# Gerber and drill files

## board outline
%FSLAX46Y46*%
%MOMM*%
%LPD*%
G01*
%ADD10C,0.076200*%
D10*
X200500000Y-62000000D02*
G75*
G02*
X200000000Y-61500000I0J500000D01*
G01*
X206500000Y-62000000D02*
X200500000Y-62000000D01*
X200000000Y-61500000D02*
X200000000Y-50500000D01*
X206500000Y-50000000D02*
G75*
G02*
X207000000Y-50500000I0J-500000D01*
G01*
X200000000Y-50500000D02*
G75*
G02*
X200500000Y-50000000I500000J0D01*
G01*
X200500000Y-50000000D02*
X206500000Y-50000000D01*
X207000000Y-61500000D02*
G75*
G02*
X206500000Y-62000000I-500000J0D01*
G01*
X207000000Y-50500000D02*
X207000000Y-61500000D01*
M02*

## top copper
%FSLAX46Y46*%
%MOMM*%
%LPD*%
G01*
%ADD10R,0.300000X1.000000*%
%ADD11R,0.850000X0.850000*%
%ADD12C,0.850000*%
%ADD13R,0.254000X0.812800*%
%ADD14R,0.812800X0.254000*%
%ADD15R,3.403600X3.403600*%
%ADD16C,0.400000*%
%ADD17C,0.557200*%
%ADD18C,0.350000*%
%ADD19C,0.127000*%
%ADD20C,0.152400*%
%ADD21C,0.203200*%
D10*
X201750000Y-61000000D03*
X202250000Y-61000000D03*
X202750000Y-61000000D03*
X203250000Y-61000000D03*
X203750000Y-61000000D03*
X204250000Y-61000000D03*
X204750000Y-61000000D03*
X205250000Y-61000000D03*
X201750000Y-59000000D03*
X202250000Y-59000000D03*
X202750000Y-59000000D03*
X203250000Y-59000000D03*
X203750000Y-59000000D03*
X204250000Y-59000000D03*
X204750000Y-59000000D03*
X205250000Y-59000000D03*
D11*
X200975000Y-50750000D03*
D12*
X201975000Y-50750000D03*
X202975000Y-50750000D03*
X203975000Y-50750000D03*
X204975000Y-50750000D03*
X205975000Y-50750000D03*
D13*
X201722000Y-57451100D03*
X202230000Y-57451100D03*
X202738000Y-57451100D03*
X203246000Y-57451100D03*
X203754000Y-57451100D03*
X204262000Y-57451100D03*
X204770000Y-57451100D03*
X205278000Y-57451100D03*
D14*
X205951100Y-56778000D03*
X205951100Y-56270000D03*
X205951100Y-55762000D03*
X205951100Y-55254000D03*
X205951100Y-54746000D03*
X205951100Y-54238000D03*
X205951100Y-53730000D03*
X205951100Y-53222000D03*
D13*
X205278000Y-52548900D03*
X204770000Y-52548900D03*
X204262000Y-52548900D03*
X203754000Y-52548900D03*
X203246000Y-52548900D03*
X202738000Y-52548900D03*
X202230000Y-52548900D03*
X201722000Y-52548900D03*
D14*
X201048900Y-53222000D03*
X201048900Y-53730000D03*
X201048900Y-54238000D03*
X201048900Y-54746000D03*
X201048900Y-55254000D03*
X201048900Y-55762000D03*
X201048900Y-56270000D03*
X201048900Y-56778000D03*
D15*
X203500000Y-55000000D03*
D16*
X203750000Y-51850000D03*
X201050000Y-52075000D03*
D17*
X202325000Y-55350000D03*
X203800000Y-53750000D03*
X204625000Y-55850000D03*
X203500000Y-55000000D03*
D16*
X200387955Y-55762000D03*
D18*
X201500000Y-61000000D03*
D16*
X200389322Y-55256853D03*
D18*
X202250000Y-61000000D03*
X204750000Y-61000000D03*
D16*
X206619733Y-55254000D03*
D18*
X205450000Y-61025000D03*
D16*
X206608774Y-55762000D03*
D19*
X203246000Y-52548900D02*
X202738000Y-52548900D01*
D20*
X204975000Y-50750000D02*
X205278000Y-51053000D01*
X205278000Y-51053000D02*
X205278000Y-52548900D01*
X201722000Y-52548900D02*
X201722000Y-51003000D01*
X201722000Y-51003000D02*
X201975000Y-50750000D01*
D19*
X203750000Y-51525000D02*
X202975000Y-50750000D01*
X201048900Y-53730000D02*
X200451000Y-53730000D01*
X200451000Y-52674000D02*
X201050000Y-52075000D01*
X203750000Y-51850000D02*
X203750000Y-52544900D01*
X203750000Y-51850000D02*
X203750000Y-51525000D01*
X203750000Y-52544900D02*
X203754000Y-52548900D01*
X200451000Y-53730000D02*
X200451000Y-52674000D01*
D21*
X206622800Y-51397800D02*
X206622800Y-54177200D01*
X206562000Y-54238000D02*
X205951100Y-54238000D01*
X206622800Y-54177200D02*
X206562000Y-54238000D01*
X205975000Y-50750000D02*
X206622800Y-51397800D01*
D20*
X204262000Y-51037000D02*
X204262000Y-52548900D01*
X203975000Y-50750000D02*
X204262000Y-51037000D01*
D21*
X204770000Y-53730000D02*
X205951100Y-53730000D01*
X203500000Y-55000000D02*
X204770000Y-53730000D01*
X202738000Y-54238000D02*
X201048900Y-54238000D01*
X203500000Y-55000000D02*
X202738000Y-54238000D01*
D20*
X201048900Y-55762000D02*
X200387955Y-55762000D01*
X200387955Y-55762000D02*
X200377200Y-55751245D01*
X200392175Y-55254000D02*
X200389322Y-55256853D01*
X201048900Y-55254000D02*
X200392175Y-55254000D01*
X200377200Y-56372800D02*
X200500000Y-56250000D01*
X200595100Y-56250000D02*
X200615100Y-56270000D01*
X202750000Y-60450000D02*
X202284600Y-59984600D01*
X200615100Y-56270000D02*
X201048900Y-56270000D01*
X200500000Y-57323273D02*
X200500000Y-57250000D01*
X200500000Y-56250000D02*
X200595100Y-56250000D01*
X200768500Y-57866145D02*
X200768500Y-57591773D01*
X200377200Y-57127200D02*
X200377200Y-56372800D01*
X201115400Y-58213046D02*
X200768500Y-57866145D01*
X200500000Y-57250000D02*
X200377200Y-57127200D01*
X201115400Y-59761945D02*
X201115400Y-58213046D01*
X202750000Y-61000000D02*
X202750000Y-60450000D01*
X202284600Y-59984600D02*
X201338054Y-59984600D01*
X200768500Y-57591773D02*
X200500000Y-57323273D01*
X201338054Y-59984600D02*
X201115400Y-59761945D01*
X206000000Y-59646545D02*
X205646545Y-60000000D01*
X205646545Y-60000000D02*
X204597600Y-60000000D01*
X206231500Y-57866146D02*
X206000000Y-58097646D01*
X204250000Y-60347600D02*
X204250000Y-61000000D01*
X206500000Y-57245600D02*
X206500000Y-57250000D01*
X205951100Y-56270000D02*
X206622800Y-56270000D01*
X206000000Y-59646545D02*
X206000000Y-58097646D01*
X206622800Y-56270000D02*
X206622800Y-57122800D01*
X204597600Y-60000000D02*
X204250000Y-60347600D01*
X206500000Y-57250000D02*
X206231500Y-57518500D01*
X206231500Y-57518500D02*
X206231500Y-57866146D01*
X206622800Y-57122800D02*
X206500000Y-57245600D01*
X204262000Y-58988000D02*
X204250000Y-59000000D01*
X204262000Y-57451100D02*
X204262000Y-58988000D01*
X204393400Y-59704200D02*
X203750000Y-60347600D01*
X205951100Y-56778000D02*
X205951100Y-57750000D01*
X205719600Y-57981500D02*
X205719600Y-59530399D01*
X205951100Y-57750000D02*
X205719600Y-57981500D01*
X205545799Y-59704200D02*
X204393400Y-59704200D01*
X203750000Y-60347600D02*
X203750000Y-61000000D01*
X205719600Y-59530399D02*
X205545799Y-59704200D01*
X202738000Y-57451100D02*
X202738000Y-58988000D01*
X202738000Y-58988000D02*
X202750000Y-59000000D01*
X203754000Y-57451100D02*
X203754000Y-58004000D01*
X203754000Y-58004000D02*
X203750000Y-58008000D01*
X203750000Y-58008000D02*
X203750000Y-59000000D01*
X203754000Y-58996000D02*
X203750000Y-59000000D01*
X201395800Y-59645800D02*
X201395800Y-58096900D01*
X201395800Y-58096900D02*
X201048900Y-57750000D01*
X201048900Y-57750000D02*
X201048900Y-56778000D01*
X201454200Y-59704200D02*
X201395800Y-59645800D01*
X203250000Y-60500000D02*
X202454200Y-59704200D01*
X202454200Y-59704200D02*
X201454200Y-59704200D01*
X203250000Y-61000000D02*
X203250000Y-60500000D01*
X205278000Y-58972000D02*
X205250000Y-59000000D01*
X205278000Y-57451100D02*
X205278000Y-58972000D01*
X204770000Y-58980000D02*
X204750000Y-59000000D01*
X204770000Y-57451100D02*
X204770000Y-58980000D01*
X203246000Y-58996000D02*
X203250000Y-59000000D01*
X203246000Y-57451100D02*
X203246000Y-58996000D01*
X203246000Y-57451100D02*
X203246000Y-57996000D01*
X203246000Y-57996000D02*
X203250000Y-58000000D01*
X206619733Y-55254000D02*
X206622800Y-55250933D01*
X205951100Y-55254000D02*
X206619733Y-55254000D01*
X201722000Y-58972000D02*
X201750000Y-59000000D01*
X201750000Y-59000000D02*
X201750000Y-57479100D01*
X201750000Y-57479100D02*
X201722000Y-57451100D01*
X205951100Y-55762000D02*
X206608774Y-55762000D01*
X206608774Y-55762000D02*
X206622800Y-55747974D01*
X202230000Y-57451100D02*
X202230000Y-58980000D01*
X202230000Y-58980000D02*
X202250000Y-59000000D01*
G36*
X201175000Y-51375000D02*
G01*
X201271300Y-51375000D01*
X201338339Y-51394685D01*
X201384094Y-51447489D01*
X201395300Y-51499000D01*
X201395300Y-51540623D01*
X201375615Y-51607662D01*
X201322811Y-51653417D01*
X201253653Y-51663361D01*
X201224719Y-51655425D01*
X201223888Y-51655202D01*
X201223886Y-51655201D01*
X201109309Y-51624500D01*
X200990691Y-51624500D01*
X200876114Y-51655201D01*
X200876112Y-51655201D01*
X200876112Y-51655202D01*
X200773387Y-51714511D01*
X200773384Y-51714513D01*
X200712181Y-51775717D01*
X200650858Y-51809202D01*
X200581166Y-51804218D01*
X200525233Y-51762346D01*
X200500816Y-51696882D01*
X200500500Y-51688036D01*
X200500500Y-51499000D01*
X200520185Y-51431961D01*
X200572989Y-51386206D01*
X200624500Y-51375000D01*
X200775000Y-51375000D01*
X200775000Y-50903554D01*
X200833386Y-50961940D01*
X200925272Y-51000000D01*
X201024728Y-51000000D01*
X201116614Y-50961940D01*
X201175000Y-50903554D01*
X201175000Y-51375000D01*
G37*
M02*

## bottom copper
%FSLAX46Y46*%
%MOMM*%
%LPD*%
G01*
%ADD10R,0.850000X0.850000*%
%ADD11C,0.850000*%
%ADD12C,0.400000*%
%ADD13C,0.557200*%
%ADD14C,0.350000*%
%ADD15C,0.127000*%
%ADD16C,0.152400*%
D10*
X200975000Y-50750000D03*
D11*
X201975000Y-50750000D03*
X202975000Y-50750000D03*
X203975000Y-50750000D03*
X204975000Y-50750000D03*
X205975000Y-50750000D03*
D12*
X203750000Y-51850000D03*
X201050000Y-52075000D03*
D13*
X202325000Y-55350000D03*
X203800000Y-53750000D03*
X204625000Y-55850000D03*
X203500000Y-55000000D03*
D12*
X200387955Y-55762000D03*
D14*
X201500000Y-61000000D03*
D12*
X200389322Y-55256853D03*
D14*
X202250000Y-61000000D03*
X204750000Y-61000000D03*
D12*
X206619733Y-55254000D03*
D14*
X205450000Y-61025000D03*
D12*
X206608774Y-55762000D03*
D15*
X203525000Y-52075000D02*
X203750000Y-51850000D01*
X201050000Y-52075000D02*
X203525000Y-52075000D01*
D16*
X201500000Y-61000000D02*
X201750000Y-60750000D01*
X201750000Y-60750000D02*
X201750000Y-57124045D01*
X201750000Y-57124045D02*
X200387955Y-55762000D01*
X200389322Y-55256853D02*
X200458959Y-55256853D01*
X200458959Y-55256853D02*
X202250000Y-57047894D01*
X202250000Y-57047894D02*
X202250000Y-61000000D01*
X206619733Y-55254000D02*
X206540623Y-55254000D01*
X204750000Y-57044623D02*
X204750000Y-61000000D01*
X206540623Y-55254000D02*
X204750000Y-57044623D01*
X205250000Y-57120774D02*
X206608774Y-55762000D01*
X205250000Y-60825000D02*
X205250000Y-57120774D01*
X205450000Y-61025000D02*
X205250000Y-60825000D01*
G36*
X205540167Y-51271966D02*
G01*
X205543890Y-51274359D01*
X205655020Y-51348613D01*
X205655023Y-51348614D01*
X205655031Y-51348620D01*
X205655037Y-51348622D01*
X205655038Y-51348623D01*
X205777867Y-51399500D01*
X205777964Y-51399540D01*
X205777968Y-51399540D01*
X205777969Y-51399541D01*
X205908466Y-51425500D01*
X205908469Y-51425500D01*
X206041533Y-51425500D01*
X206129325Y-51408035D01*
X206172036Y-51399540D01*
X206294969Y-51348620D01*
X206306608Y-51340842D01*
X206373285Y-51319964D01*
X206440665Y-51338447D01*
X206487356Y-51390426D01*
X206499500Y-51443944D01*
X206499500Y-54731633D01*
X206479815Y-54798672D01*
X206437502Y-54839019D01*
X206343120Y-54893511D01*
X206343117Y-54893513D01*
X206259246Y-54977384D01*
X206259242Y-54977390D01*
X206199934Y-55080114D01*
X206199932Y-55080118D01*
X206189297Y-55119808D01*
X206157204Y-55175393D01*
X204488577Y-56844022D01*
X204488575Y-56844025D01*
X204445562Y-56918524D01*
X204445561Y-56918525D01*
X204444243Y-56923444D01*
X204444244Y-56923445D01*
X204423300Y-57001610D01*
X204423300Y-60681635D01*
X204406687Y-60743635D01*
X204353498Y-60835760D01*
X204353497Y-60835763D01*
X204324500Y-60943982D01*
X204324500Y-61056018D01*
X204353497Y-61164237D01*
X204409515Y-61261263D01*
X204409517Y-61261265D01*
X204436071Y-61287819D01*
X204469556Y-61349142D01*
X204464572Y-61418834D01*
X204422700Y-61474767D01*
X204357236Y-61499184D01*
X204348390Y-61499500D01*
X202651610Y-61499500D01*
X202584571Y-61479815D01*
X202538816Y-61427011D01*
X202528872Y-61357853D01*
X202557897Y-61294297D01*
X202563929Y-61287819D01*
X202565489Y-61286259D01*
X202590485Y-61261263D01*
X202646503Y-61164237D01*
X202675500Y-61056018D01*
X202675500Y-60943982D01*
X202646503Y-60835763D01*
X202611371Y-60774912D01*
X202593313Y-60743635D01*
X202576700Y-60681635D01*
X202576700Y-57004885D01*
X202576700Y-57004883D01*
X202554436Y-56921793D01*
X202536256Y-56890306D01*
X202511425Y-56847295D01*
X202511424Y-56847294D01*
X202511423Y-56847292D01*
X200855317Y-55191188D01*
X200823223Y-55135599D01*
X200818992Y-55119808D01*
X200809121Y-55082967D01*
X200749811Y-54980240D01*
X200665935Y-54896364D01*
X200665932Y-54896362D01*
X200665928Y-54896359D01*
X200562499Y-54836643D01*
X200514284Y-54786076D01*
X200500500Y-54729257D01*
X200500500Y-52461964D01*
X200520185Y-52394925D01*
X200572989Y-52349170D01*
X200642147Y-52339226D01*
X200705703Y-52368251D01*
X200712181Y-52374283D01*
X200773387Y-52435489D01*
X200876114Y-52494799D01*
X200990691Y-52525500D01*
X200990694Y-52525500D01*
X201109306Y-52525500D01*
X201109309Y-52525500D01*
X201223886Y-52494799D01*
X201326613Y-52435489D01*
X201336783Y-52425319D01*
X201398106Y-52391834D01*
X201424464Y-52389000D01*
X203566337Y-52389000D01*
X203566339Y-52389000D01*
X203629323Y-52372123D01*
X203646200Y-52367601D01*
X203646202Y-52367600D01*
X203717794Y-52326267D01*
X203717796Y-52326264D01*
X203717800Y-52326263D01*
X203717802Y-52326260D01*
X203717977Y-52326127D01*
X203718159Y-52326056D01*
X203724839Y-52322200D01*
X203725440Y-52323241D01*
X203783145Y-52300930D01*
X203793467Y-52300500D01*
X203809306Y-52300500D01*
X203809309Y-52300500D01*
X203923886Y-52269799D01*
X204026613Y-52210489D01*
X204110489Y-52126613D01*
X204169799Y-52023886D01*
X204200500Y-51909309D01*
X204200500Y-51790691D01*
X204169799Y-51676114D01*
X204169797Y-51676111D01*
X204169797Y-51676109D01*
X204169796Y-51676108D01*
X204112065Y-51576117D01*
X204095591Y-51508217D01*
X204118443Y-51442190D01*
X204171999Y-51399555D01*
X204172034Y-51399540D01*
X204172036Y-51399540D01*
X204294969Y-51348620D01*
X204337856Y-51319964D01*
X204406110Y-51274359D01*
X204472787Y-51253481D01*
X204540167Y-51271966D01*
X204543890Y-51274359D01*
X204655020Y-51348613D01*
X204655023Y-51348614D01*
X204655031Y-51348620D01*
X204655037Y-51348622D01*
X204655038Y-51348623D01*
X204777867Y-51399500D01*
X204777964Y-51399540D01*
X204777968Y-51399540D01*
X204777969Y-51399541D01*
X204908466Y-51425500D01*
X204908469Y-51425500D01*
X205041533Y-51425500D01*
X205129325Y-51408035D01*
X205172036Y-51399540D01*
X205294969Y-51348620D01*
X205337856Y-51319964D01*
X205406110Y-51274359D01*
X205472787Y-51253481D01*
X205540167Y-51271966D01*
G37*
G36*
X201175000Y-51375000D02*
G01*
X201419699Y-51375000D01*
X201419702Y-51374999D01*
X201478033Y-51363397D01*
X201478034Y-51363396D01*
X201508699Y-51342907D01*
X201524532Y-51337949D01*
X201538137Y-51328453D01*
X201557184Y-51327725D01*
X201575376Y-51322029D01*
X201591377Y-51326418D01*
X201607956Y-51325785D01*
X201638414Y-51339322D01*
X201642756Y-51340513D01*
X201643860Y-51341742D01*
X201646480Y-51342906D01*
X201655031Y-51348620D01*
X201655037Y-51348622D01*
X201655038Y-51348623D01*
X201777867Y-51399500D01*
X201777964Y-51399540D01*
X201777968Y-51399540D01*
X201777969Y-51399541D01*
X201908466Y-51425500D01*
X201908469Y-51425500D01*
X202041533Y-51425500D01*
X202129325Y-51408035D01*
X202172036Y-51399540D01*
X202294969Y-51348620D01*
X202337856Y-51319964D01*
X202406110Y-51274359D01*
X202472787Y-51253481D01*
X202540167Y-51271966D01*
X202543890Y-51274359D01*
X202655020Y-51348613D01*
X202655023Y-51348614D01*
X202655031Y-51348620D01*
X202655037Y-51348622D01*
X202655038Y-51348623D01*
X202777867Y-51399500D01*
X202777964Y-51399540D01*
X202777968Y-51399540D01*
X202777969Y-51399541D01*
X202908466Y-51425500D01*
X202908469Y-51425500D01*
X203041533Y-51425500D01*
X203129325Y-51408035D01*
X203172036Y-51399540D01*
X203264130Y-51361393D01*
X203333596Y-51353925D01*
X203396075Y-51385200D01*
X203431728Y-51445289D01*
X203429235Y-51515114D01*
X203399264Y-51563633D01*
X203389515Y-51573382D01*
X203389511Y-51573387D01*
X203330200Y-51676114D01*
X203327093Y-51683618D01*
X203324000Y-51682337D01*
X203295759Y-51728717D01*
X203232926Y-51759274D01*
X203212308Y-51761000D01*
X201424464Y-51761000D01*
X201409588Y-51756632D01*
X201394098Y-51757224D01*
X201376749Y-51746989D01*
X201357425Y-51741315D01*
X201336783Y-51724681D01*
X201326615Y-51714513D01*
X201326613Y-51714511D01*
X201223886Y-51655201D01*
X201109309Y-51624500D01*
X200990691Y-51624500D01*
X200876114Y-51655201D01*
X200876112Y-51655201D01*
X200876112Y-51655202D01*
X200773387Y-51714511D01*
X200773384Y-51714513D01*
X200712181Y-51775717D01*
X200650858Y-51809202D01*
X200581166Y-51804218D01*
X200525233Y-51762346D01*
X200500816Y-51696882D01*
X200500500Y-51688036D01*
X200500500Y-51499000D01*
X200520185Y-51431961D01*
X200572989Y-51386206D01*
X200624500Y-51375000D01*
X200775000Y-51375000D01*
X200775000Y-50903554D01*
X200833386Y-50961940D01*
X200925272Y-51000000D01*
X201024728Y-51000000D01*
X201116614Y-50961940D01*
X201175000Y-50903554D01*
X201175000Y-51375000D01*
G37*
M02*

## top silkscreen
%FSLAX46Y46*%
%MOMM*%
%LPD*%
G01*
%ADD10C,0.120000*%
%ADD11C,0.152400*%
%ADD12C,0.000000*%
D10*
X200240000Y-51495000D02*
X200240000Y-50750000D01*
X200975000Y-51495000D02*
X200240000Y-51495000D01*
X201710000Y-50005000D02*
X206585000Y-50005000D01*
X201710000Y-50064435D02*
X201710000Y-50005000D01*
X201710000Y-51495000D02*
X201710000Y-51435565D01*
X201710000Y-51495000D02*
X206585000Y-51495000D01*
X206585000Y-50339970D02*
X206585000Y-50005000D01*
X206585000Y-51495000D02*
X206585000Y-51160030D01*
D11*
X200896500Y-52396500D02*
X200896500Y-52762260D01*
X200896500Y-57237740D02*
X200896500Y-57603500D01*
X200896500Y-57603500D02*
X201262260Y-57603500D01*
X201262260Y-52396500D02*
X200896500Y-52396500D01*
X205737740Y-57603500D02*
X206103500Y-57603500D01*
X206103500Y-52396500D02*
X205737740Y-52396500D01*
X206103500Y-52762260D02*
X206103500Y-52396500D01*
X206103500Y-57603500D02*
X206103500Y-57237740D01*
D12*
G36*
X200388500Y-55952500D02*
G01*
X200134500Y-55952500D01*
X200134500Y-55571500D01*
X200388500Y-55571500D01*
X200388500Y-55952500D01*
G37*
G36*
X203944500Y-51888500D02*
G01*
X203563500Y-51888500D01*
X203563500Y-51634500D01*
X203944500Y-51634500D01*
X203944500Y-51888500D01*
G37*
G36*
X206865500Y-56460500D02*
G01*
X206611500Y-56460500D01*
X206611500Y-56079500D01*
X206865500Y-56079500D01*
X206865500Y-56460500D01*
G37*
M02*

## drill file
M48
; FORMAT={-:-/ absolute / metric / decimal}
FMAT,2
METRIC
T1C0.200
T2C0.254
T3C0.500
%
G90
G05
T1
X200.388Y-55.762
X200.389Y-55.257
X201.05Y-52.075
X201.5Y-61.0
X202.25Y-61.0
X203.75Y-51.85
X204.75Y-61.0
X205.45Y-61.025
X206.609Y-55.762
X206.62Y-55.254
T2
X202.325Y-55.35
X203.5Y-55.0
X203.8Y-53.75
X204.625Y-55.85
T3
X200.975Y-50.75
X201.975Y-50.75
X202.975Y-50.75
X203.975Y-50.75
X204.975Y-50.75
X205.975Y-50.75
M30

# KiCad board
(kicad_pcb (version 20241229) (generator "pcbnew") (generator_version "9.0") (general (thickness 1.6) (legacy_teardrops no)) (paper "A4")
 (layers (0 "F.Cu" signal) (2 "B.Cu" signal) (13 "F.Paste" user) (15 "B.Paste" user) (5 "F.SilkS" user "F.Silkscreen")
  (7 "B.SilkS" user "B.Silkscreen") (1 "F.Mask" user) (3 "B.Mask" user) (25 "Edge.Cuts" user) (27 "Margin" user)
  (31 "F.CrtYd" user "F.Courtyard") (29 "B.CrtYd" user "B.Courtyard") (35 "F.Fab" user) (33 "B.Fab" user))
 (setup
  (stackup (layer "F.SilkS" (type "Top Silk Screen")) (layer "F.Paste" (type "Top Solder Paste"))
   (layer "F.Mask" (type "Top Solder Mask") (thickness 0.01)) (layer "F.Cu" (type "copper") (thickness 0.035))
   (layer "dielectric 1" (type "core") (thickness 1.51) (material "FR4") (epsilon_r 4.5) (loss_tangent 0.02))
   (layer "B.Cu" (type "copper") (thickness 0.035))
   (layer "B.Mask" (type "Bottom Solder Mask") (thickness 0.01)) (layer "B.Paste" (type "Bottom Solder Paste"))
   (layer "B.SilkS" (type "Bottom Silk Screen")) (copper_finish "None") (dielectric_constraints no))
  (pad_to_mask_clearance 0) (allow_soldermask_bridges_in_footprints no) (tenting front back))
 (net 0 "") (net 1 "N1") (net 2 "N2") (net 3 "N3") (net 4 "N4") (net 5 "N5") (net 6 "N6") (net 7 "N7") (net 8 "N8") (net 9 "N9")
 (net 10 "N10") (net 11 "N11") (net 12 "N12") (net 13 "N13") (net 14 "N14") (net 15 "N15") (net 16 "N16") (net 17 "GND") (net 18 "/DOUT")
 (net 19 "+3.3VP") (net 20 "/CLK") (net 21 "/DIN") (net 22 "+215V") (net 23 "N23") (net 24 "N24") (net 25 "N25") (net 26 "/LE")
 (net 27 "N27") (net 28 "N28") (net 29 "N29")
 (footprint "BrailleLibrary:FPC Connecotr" (layer "F.Cu") (at 203.5 61 90)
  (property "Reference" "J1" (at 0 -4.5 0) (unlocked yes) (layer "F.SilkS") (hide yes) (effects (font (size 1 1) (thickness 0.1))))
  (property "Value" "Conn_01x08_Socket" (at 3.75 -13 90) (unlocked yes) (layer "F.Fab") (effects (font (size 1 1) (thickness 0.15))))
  (pad "1" smd rect (at 0 -1.75 90) (size 1 0.3) (layers "F.Cu" "F.Mask" "F.Paste") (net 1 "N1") (thermal_bridge_angle 45))
  (pad "2" smd rect (at 0 -1.25 90) (size 1 0.3) (layers "F.Cu" "F.Mask" "F.Paste") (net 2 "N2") (thermal_bridge_angle 45))
  (pad "3" smd rect (at 0 -0.75 90) (size 1 0.3) (layers "F.Cu" "F.Mask" "F.Paste") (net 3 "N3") (thermal_bridge_angle 45))
  (pad "4" smd rect (at 0 -0.25 90) (size 1 0.3) (layers "F.Cu" "F.Mask" "F.Paste") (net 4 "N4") (thermal_bridge_angle 45))
  (pad "5" smd rect (at 0 0.25 90) (size 1 0.3) (layers "F.Cu" "F.Mask" "F.Paste") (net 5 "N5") (thermal_bridge_angle 45))
  (pad "6" smd rect (at 0 0.75 90) (size 1 0.3) (layers "F.Cu" "F.Mask" "F.Paste") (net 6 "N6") (thermal_bridge_angle 45))
  (pad "7" smd rect (at 0 1.25 90) (size 1 0.3) (layers "F.Cu" "F.Mask" "F.Paste") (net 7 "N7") (thermal_bridge_angle 45))
  (pad "8" smd rect (at 0 1.75 90) (size 1 0.3) (layers "F.Cu" "F.Mask" "F.Paste") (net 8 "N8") (thermal_bridge_angle 45)))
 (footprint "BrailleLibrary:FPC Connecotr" (layer "F.Cu") (at 203.5 59 90)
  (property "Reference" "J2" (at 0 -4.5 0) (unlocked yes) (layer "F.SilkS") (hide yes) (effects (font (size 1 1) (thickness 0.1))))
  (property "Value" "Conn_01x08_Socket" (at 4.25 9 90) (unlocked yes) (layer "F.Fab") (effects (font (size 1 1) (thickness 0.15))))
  (pad "1" smd rect (at 0 -1.75 90) (size 1 0.3) (layers "F.Cu" "F.Mask" "F.Paste") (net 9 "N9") (thermal_bridge_angle 45))
  (pad "2" smd rect (at 0 -1.25 90) (size 1 0.3) (layers "F.Cu" "F.Mask" "F.Paste") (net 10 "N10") (thermal_bridge_angle 45))
  (pad "3" smd rect (at 0 -0.75 90) (size 1 0.3) (layers "F.Cu" "F.Mask" "F.Paste") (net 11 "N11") (thermal_bridge_angle 45))
  (pad "4" smd rect (at 0 -0.25 90) (size 1 0.3) (layers "F.Cu" "F.Mask" "F.Paste") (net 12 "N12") (thermal_bridge_angle 45))
  (pad "5" smd rect (at 0 0.25 90) (size 1 0.3) (layers "F.Cu" "F.Mask" "F.Paste") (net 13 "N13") (thermal_bridge_angle 45))
  (pad "6" smd rect (at 0 0.75 90) (size 1 0.3) (layers "F.Cu" "F.Mask" "F.Paste") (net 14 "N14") (thermal_bridge_angle 45))
  (pad "7" smd rect (at 0 1.25 90) (size 1 0.3) (layers "F.Cu" "F.Mask" "F.Paste") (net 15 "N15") (thermal_bridge_angle 45))
  (pad "8" smd rect (at 0 1.75 90) (size 1 0.3) (layers "F.Cu" "F.Mask" "F.Paste") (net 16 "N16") (thermal_bridge_angle 45)))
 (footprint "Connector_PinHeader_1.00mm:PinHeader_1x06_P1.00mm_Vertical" (layer "F.Cu") (at 200.975 50.75 90)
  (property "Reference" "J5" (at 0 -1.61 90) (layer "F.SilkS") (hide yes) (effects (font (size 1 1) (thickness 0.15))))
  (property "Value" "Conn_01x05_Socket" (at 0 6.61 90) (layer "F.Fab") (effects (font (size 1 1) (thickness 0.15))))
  (fp_line (start -0.745 -0.735) (end 0 -0.735) (stroke (width 0.12) (type solid)) (layer "F.SilkS"))
  (fp_line (start -0.745 0) (end -0.745 -0.735) (stroke (width 0.12) (type solid)) (layer "F.SilkS"))
  (fp_line (start 0.745 0.735) (end 0.745 5.61) (stroke (width 0.12) (type solid)) (layer "F.SilkS"))
  (fp_line (start 0.685565 0.735) (end 0.745 0.735) (stroke (width 0.12) (type solid)) (layer "F.SilkS"))
  (fp_line (start -0.745 0.735) (end -0.685565 0.735) (stroke (width 0.12) (type solid)) (layer "F.SilkS"))
  (fp_line (start -0.745 0.735) (end -0.745 5.61) (stroke (width 0.12) (type solid)) (layer "F.SilkS"))
  (fp_line (start 0.41003 5.61) (end 0.745 5.61) (stroke (width 0.12) (type solid)) (layer "F.SilkS"))
  (fp_line (start -0.745 5.61) (end -0.41003 5.61) (stroke (width 0.12) (type solid)) (layer "F.SilkS"))
  (pad "1" thru_hole rect (at 0 0 90) (size 0.85 0.85) (drill 0.5) (layers "*.Cu" "*.Mask") (remove_unused_layers no) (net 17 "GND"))
  (pad "2" thru_hole circle (at 0 1 90) (size 0.85 0.85) (drill 0.5) (layers "*.Cu" "*.Mask") (remove_unused_layers no) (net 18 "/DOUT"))
  (pad "3" thru_hole circle (at 0 2 90) (size 0.85 0.85) (drill 0.5) (layers "*.Cu" "*.Mask") (remove_unused_layers no) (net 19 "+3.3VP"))
  (pad "4" thru_hole circle (at 0 3 90) (size 0.85 0.85) (drill 0.5) (layers "*.Cu" "*.Mask") (remove_unused_layers no) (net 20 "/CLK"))
  (pad "5" thru_hole circle (at 0 4 90) (size 0.85 0.85) (drill 0.5) (layers "*.Cu" "*.Mask") (remove_unused_layers no) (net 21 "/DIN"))
  (pad "6" thru_hole circle (at 0 5 90) (size 0.85 0.85) (drill 0.5) (layers "*.Cu" "*.Mask") (remove_unused_layers no) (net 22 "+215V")))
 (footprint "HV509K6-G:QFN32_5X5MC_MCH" (layer "F.Cu") (at 203.5 55 90)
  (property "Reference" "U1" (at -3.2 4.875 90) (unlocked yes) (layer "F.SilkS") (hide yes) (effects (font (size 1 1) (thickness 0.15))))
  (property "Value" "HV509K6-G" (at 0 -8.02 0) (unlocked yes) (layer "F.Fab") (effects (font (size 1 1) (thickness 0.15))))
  (fp_line (start 2.6035 -2.6035) (end 2.23774 -2.6035) (stroke (width 0.1524) (type solid)) (layer "F.SilkS"))
  (fp_line (start -2.23774 -2.6035) (end -2.6035 -2.6035) (stroke (width 0.1524) (type solid)) (layer "F.SilkS"))
  (fp_line (start -2.6035 -2.6035) (end -2.6035 -2.23774) (stroke (width 0.1524) (type solid)) (layer "F.SilkS"))
  (fp_line (start 2.6035 -2.23774) (end 2.6035 -2.6035) (stroke (width 0.1524) (type solid)) (layer "F.SilkS"))
  (fp_line (start -2.6035 2.23774) (end -2.6035 2.6035) (stroke (width 0.1524) (type solid)) (layer "F.SilkS"))
  (fp_line (start 2.6035 2.6035) (end 2.6035 2.23774) (stroke (width 0.1524) (type solid)) (layer "F.SilkS"))
  (fp_line (start 2.23774 2.6035) (end 2.6035 2.6035) (stroke (width 0.1524) (type solid)) (layer "F.SilkS"))
  (fp_line (start -2.6035 2.6035) (end -2.23774 2.6035) (stroke (width 0.1524) (type solid)) (layer "F.SilkS"))
  (fp_poly
   (pts (xy -0.9525 -3.1115) (xy -0.9525 -3.3655) (xy -0.5715 -3.3655) (xy -0.5715 -3.1115)) (stroke (width 0) (type solid)) (fill yes)
   (layer "F.SilkS"))
  (fp_poly
   (pts (xy 3.3655 0.0635) (xy 3.3655 0.4445) (xy 3.1115 0.4445) (xy 3.1115 0.0635)) (stroke (width 0) (type solid)) (fill yes)
   (layer "F.SilkS"))
  (fp_poly
   (pts (xy -1.4605 3.1115) (xy -1.4605 3.3655) (xy -1.0795 3.3655) (xy -1.0795 3.1115)) (stroke (width 0) (type solid)) (fill yes)
   (layer "F.SilkS"))
  (pad "1" smd rect (at -2.4511 -1.778 180) (size 0.254 0.8128) (layers "F.Cu" "F.Mask" "F.Paste") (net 9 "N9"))
  (pad "2" smd rect (at -2.4511 -1.27 180) (size 0.254 0.8128) (layers "F.Cu" "F.Mask" "F.Paste") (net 10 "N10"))
  (pad "3" smd rect (at -2.4511 -0.762 180) (size 0.254 0.8128) (layers "F.Cu" "F.Mask" "F.Paste") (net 11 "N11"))
  (pad "4" smd rect (at -2.4511 -0.254 180) (size 0.254 0.8128) (layers "F.Cu" "F.Mask" "F.Paste") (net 12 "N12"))
  (pad "5" smd rect (at -2.4511 0.254 180) (size 0.254 0.8128) (layers "F.Cu" "F.Mask" "F.Paste") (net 13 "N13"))
  (pad "6" smd rect (at -2.4511 0.762 180) (size 0.254 0.8128) (layers "F.Cu" "F.Mask" "F.Paste") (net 14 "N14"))
  (pad "7" smd rect (at -2.4511 1.27 180) (size 0.254 0.8128) (layers "F.Cu" "F.Mask" "F.Paste") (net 15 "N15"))
  (pad "8" smd rect (at -2.4511 1.778 180) (size 0.254 0.8128) (layers "F.Cu" "F.Mask" "F.Paste") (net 16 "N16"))
  (pad "9" smd rect (at -1.778 2.4511 90) (size 0.254 0.8128) (layers "F.Cu" "F.Mask" "F.Paste") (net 5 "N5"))
  (pad "10" smd rect (at -1.27 2.4511 90) (size 0.254 0.8128) (layers "F.Cu" "F.Mask" "F.Paste") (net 6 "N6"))
  (pad "11" smd rect (at -0.762 2.4511 90) (size 0.254 0.8128) (layers "F.Cu" "F.Mask" "F.Paste") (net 8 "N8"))
  (pad "12" smd rect (at -0.254 2.4511 90) (size 0.254 0.8128) (layers "F.Cu" "F.Mask" "F.Paste") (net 7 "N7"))
  (pad "13" smd rect (at 0.254 2.4511 90) (size 0.254 0.8128) (layers "F.Cu" "F.Mask" "F.Paste") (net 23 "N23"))
  (pad "14" smd rect (at 0.762 2.4511 90) (size 0.254 0.8128) (layers "F.Cu" "F.Mask" "F.Paste") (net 22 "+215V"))
  (pad "15" smd rect (at 1.27 2.4511 90) (size 0.254 0.8128) (layers "F.Cu" "F.Mask" "F.Paste") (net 17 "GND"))
  (pad "16" smd rect (at 1.778 2.4511 90) (size 0.254 0.8128) (layers "F.Cu" "F.Mask" "F.Paste") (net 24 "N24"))
  (pad "17" smd rect (at 2.4511 1.778 180) (size 0.254 0.8128) (layers "F.Cu" "F.Mask" "F.Paste") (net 21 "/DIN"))
  (pad "18" smd rect (at 2.4511 1.27 180) (size 0.254 0.8128) (layers "F.Cu" "F.Mask" "F.Paste") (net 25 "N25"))
  (pad "19" smd rect (at 2.4511 0.762 180) (size 0.254 0.8128) (layers "F.Cu" "F.Mask" "F.Paste") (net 20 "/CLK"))
  (pad "20" smd rect (at 2.4511 0.254 180) (size 0.254 0.8128) (layers "F.Cu" "F.Mask" "F.Paste") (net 19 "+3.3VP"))
  (pad "21" smd rect (at 2.4511 -0.254 180) (size 0.254 0.8128) (layers "F.Cu" "F.Mask" "F.Paste") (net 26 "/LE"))
  (pad "22" smd rect (at 2.4511 -0.762 180) (size 0.254 0.8128) (layers "F.Cu" "F.Mask" "F.Paste") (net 26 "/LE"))
  (pad "23" smd rect (at 2.4511 -1.27 180) (size 0.254 0.8128) (layers "F.Cu" "F.Mask" "F.Paste") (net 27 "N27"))
  (pad "24" smd rect (at 2.4511 -1.778 180) (size 0.254 0.8128) (layers "F.Cu" "F.Mask" "F.Paste") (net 18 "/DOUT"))
  (pad "25" smd rect (at 1.778 -2.4511 90) (size 0.254 0.8128) (layers "F.Cu" "F.Mask" "F.Paste") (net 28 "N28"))
  (pad "26" smd rect (at 1.27 -2.4511 90) (size 0.254 0.8128) (layers "F.Cu" "F.Mask" "F.Paste") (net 19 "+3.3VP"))
  (pad "27" smd rect (at 0.762 -2.4511 90) (size 0.254 0.8128) (layers "F.Cu" "F.Mask" "F.Paste") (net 17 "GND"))
  (pad "28" smd rect (at 0.254 -2.4511 90) (size 0.254 0.8128) (layers "F.Cu" "F.Mask" "F.Paste") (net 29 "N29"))
  (pad "29" smd rect (at -0.254 -2.4511 90) (size 0.254 0.8128) (layers "F.Cu" "F.Mask" "F.Paste") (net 2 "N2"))
  (pad "30" smd rect (at -0.762 -2.4511 90) (size 0.254 0.8128) (layers "F.Cu" "F.Mask" "F.Paste") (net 1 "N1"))
  (pad "31" smd rect (at -1.27 -2.4511 90) (size 0.254 0.8128) (layers "F.Cu" "F.Mask" "F.Paste") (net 3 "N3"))
  (pad "32" smd rect (at -1.778 -2.4511 90) (size 0.254 0.8128) (layers "F.Cu" "F.Mask" "F.Paste") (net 4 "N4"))
  (pad "33" smd rect (at 0 0 90) (size 3.4036 3.4036) (layers "F.Cu" "F.Mask" "F.Paste") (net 17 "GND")))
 (gr_arc (start 200.5 62) (mid 200.146447 61.853553) (end 200 61.5) (stroke (width 0.0762) (type default)) (layer "Edge.Cuts"))
 (gr_line (start 206.5 62) (end 200.5 62) (stroke (width 0.0762) (type default)) (layer "Edge.Cuts"))
 (gr_line (start 200 61.5) (end 200 50.5) (stroke (width 0.0762) (type default)) (layer "Edge.Cuts"))
 (gr_arc (start 206.5 50) (mid 206.853553 50.146447) (end 207 50.5) (stroke (width 0.0762) (type default)) (layer "Edge.Cuts"))
 (gr_arc (start 200 50.5) (mid 200.146447 50.146447) (end 200.5 50) (stroke (width 0.0762) (type default)) (layer "Edge.Cuts"))
 (gr_line (start 200.5 50) (end 206.5 50) (stroke (width 0.0762) (type default)) (layer "Edge.Cuts"))
 (gr_arc (start 207 61.5) (mid 206.853553 61.853553) (end 206.5 62) (stroke (width 0.0762) (type default)) (layer "Edge.Cuts"))
 (gr_line (start 207 50.5) (end 207 61.5) (stroke (width 0.0762) (type default)) (layer "Edge.Cuts"))
 (segment (start 203.246 52.5489) (end 202.738 52.5489) (width 0.127) (layer "F.Cu") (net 26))
 (segment (start 204.975 50.75) (end 205.278 51.053) (width 0.1524) (layer "F.Cu") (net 21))
 (segment (start 205.278 51.053) (end 205.278 52.5489) (width 0.1524) (layer "F.Cu") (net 21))
 (segment (start 201.722 52.5489) (end 201.722 51.003) (width 0.1524) (layer "F.Cu") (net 18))
 (segment (start 201.722 51.003) (end 201.975 50.75) (width 0.1524) (layer "F.Cu") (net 18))
 (segment (start 203.75 51.525) (end 202.975 50.75) (width 0.127) (layer "F.Cu") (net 19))
 (segment (start 201.0489 53.73) (end 200.451 53.73) (width 0.127) (layer "F.Cu") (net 19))
 (segment (start 200.451 52.674) (end 201.05 52.075) (width 0.127) (layer "F.Cu") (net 19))
 (segment (start 203.75 51.85) (end 203.75 52.5449) (width 0.127) (layer "F.Cu") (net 19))
 (segment (start 203.75 51.85) (end 203.75 51.525) (width 0.127) (layer "F.Cu") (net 19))
 (segment (start 203.75 52.5449) (end 203.754 52.5489) (width 0.127) (layer "F.Cu") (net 19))
 (segment (start 200.451 53.73) (end 200.451 52.674) (width 0.127) (layer "F.Cu") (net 19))
 (via (at 203.75 51.85) (size 0.4) (drill 0.2) (layers "F.Cu" "B.Cu") (free yes) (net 19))
 (via (at 201.05 52.075) (size 0.4) (drill 0.2) (layers "F.Cu" "B.Cu") (free yes) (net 19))
 (segment (start 203.525 52.075) (end 203.75 51.85) (width 0.127) (layer "B.Cu") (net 19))
 (segment (start 201.05 52.075) (end 203.525 52.075) (width 0.127) (layer "B.Cu") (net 19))
 (segment (start 206.6228 51.3978) (end 206.6228 54.1772) (width 0.2032) (layer "F.Cu") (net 22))
 (segment (start 206.562 54.238) (end 205.9511 54.238) (width 0.2032) (layer "F.Cu") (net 22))
 (segment (start 206.6228 54.1772) (end 206.562 54.238) (width 0.2032) (layer "F.Cu") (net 22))
 (segment (start 205.975 50.75) (end 206.6228 51.3978) (width 0.2032) (layer "F.Cu") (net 22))
 (segment (start 204.262 51.037) (end 204.262 52.5489) (width 0.1524) (layer "F.Cu") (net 20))
 (segment (start 203.975 50.75) (end 204.262 51.037) (width 0.1524) (layer "F.Cu") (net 20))
 (segment (start 204.77 53.73) (end 205.9511 53.73) (width 0.2032) (layer "F.Cu") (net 17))
 (segment (start 203.5 55) (end 204.77 53.73) (width 0.2032) (layer "F.Cu") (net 17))
 (segment (start 202.738 54.238) (end 201.0489 54.238) (width 0.2032) (layer "F.Cu") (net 17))
 (segment (start 203.5 55) (end 202.738 54.238) (width 0.2032) (layer "F.Cu") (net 17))
 (via (at 202.325 55.35) (size 0.5572) (drill 0.254) (layers "F.Cu" "B.Cu") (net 17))
 (via (at 203.8 53.75) (size 0.5572) (drill 0.254) (layers "F.Cu" "B.Cu") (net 17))
 (via (at 204.625 55.85) (size 0.5572) (drill 0.254) (layers "F.Cu" "B.Cu") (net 17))
 (via (at 203.5 55) (size 0.5572) (drill 0.254) (layers "F.Cu" "B.Cu") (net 17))
 (segment (start 201.0489 55.762) (end 200.387955 55.762) (width 0.1524) (layer "F.Cu") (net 1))
 (segment (start 200.387955 55.762) (end 200.3772 55.751245) (width 0.1524) (layer "F.Cu") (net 1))
 (via (at 200.387955 55.762) (size 0.4) (drill 0.2) (layers "F.Cu" "B.Cu") (free yes) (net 1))
 (via (at 201.5 61) (size 0.35) (drill 0.2) (layers "F.Cu" "B.Cu") (free yes) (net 1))
 (segment (start 201.5 61) (end 201.75 60.75) (width 0.1524) (layer "B.Cu") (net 1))
 (segment (start 201.75 60.75) (end 201.75 57.124045) (width 0.1524) (layer "B.Cu") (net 1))
 (segment (start 201.75 57.124045) (end 200.387955 55.762) (width 0.1524) (layer "B.Cu") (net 1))
 (segment (start 200.392175 55.254) (end 200.389322 55.256853) (width 0.1524) (layer "F.Cu") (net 2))
 (segment (start 201.0489 55.254) (end 200.392175 55.254) (width 0.1524) (layer "F.Cu") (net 2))
 (via (at 200.389322 55.256853) (size 0.4) (drill 0.2) (layers "F.Cu" "B.Cu") (free yes) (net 2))
 (via (at 202.25 61) (size 0.35) (drill 0.2) (layers "F.Cu" "B.Cu") (free yes) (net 2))
 (segment (start 200.389322 55.256853) (end 200.458959 55.256853) (width 0.1524) (layer "B.Cu") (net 2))
 (segment (start 200.458959 55.256853) (end 202.25 57.047894) (width 0.1524) (layer "B.Cu") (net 2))
 (segment (start 202.25 57.047894) (end 202.25 61) (width 0.1524) (layer "B.Cu") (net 2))
 (segment (start 200.3772 56.3728) (end 200.5 56.25) (width 0.1524) (layer "F.Cu") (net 3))
 (segment (start 200.5951 56.25) (end 200.6151 56.27) (width 0.1524) (layer "F.Cu") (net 3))
 (segment (start 202.75 60.45) (end 202.2846 59.9846) (width 0.1524) (layer "F.Cu") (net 3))
 (segment (start 200.6151 56.27) (end 201.0489 56.27) (width 0.1524) (layer "F.Cu") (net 3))
 (segment (start 200.5 57.323273) (end 200.5 57.25) (width 0.1524) (layer "F.Cu") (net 3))
 (segment (start 200.5 56.25) (end 200.5951 56.25) (width 0.1524) (layer "F.Cu") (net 3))
 (segment (start 200.7685 57.866145) (end 200.7685 57.591773) (width 0.1524) (layer "F.Cu") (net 3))
 (segment (start 200.3772 57.1272) (end 200.3772 56.3728) (width 0.1524) (layer "F.Cu") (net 3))
 (segment (start 201.1154 58.213046) (end 200.7685 57.866145) (width 0.1524) (layer "F.Cu") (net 3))
 (segment (start 200.5 57.25) (end 200.3772 57.1272) (width 0.1524) (layer "F.Cu") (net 3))
 (segment (start 201.1154 59.761945) (end 201.1154 58.213046) (width 0.1524) (layer "F.Cu") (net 3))
 (segment (start 202.75 61) (end 202.75 60.45) (width 0.1524) (layer "F.Cu") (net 3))
 (segment (start 202.2846 59.9846) (end 201.338054 59.9846) (width 0.1524) (layer "F.Cu") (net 3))
 (segment (start 200.7685 57.591773) (end 200.5 57.323273) (width 0.1524) (layer "F.Cu") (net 3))
 (segment (start 201.338054 59.9846) (end 201.1154 59.761945) (width 0.1524) (layer "F.Cu") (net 3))
 (segment (start 206 59.646545) (end 205.646545 60) (width 0.1524) (layer "F.Cu") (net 6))
 (segment (start 205.646545 60) (end 204.5976 60) (width 0.1524) (layer "F.Cu") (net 6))
 (segment (start 206.2315 57.866146) (end 206 58.097646) (width 0.1524) (layer "F.Cu") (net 6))
 (segment (start 204.25 60.3476) (end 204.25 61) (width 0.1524) (layer "F.Cu") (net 6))
 (segment (start 206.5 57.2456) (end 206.5 57.25) (width 0.1524) (layer "F.Cu") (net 6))
 (segment (start 205.9511 56.27) (end 206.6228 56.27) (width 0.1524) (layer "F.Cu") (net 6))
 (segment (start 206 59.646545) (end 206 58.097646) (width 0.1524) (layer "F.Cu") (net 6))
 (segment (start 206.6228 56.27) (end 206.6228 57.1228) (width 0.1524) (layer "F.Cu") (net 6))
 (segment (start 204.5976 60) (end 204.25 60.3476) (width 0.1524) (layer "F.Cu") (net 6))
 (segment (start 206.5 57.25) (end 206.2315 57.5185) (width 0.1524) (layer "F.Cu") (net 6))
 (segment (start 206.2315 57.5185) (end 206.2315 57.866146) (width 0.1524) (layer "F.Cu") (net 6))
 (segment (start 206.6228 57.1228) (end 206.5 57.2456) (width 0.1524) (layer "F.Cu") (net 6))
 (segment (start 204.262 58.988) (end 204.25 59) (width 0.1524) (layer "F.Cu") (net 14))
 (segment (start 204.262 57.4511) (end 204.262 58.988) (width 0.1524) (layer "F.Cu") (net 14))
 (segment (start 204.3934 59.7042) (end 203.75 60.3476) (width 0.1524) (layer "F.Cu") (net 5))
 (segment (start 205.9511 56.778) (end 205.9511 57.75) (width 0.1524) (layer "F.Cu") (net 5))
 (segment (start 205.7196 57.9815) (end 205.7196 59.530399) (width 0.1524) (layer "F.Cu") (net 5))
 (segment (start 205.9511 57.75) (end 205.7196 57.9815) (width 0.1524) (layer "F.Cu") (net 5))
 (segment (start 205.545799 59.7042) (end 204.3934 59.7042) (width 0.1524) (layer "F.Cu") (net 5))
 (segment (start 203.75 60.3476) (end 203.75 61) (width 0.1524) (layer "F.Cu") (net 5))
 (segment (start 205.7196 59.530399) (end 205.545799 59.7042) (width 0.1524) (layer "F.Cu") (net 5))
 (segment (start 202.738 57.4511) (end 202.738 58.988) (width 0.1524) (layer "F.Cu") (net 11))
 (segment (start 202.738 58.988) (end 202.75 59) (width 0.1524) (layer "F.Cu") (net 11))
 (segment (start 203.754 57.4511) (end 203.754 58.004) (width 0.1524) (layer "F.Cu") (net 13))
 (segment (start 203.754 58.004) (end 203.75 58.008) (width 0.1524) (layer "F.Cu") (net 13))
 (segment (start 203.75 58.008) (end 203.75 59) (width 0.1524) (layer "F.Cu") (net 13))
 (segment (start 203.754 58.996) (end 203.75 59) (width 0.1524) (layer "F.Cu") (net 13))
 (segment (start 201.3958 59.6458) (end 201.3958 58.0969) (width 0.1524) (layer "F.Cu") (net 4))
 (segment (start 201.3958 58.0969) (end 201.0489 57.75) (width 0.1524) (layer "F.Cu") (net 4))
 (segment (start 201.0489 57.75) (end 201.0489 56.778) (width 0.1524) (layer "F.Cu") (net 4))
 (segment (start 201.4542 59.7042) (end 201.3958 59.6458) (width 0.1524) (layer "F.Cu") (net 4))
 (segment (start 203.25 60.5) (end 202.4542 59.7042) (width 0.1524) (layer "F.Cu") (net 4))
 (segment (start 202.4542 59.7042) (end 201.4542 59.7042) (width 0.1524) (layer "F.Cu") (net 4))
 (segment (start 203.25 61) (end 203.25 60.5) (width 0.1524) (layer "F.Cu") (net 4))
 (segment (start 205.278 58.972) (end 205.25 59) (width 0.1524) (layer "F.Cu") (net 16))
 (segment (start 205.278 57.4511) (end 205.278 58.972) (width 0.1524) (layer "F.Cu") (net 16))
 (segment (start 204.77 58.98) (end 204.75 59) (width 0.1524) (layer "F.Cu") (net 15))
 (segment (start 204.77 57.4511) (end 204.77 58.98) (width 0.1524) (layer "F.Cu") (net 15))
 (segment (start 203.246 58.996) (end 203.25 59) (width 0.1524) (layer "F.Cu") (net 12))
 (segment (start 203.246 57.4511) (end 203.246 58.996) (width 0.1524) (layer "F.Cu") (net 12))
 (segment (start 203.246 57.4511) (end 203.246 57.996) (width 0.1524) (layer "F.Cu") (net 12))
 (segment (start 203.246 57.996) (end 203.25 58) (width 0.1524) (layer "F.Cu") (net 12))
 (segment (start 206.619733 55.254) (end 206.6228 55.250933) (width 0.1524) (layer "F.Cu") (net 7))
 (segment (start 205.9511 55.254) (end 206.619733 55.254) (width 0.1524) (layer "F.Cu") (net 7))
 (via (at 204.75 61) (size 0.35) (drill 0.2) (layers "F.Cu" "B.Cu") (free yes) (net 7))
 (via (at 206.619733 55.254) (size 0.4) (drill 0.2) (layers "F.Cu" "B.Cu") (free yes) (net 7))
 (segment (start 206.619733 55.254) (end 206.540623 55.254) (width 0.1524) (layer "B.Cu") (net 7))
 (segment (start 204.75 57.044623) (end 204.75 61) (width 0.1524) (layer "B.Cu") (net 7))
 (segment (start 206.540623 55.254) (end 204.75 57.044623) (width 0.1524) (layer "B.Cu") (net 7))
 (segment (start 201.722 58.972) (end 201.75 59) (width 0.1524) (layer "F.Cu") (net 9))
 (segment (start 201.75 59) (end 201.75 57.4791) (width 0.1524) (layer "F.Cu") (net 9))
 (segment (start 201.75 57.4791) (end 201.722 57.4511) (width 0.1524) (layer "F.Cu") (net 9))
 (segment (start 205.9511 55.762) (end 206.608774 55.762) (width 0.1524) (layer "F.Cu") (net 8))
 (segment (start 206.608774 55.762) (end 206.6228 55.747974) (width 0.1524) (layer "F.Cu") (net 8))
 (via (at 205.45 61.025) (size 0.35) (drill 0.2) (layers "F.Cu" "B.Cu") (free yes) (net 8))
 (via (at 206.608774 55.762) (size 0.4) (drill 0.2) (layers "F.Cu" "B.Cu") (free yes) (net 8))
 (segment (start 205.25 57.120774) (end 206.608774 55.762) (width 0.1524) (layer "B.Cu") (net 8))
 (segment (start 205.25 60.825) (end 205.25 57.120774) (width 0.1524) (layer "B.Cu") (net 8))
 (segment (start 205.45 61.025) (end 205.25 60.825) (width 0.1524) (layer "B.Cu") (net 8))
 (segment (start 202.23 57.4511) (end 202.23 58.98) (width 0.1524) (layer "F.Cu") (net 10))
 (segment (start 202.23 58.98) (end 202.25 59) (width 0.1524) (layer "F.Cu") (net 10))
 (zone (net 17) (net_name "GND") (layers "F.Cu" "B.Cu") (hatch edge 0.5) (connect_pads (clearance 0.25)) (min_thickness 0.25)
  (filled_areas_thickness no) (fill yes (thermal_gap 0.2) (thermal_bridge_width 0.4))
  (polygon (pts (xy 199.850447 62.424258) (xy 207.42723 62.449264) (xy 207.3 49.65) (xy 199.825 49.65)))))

